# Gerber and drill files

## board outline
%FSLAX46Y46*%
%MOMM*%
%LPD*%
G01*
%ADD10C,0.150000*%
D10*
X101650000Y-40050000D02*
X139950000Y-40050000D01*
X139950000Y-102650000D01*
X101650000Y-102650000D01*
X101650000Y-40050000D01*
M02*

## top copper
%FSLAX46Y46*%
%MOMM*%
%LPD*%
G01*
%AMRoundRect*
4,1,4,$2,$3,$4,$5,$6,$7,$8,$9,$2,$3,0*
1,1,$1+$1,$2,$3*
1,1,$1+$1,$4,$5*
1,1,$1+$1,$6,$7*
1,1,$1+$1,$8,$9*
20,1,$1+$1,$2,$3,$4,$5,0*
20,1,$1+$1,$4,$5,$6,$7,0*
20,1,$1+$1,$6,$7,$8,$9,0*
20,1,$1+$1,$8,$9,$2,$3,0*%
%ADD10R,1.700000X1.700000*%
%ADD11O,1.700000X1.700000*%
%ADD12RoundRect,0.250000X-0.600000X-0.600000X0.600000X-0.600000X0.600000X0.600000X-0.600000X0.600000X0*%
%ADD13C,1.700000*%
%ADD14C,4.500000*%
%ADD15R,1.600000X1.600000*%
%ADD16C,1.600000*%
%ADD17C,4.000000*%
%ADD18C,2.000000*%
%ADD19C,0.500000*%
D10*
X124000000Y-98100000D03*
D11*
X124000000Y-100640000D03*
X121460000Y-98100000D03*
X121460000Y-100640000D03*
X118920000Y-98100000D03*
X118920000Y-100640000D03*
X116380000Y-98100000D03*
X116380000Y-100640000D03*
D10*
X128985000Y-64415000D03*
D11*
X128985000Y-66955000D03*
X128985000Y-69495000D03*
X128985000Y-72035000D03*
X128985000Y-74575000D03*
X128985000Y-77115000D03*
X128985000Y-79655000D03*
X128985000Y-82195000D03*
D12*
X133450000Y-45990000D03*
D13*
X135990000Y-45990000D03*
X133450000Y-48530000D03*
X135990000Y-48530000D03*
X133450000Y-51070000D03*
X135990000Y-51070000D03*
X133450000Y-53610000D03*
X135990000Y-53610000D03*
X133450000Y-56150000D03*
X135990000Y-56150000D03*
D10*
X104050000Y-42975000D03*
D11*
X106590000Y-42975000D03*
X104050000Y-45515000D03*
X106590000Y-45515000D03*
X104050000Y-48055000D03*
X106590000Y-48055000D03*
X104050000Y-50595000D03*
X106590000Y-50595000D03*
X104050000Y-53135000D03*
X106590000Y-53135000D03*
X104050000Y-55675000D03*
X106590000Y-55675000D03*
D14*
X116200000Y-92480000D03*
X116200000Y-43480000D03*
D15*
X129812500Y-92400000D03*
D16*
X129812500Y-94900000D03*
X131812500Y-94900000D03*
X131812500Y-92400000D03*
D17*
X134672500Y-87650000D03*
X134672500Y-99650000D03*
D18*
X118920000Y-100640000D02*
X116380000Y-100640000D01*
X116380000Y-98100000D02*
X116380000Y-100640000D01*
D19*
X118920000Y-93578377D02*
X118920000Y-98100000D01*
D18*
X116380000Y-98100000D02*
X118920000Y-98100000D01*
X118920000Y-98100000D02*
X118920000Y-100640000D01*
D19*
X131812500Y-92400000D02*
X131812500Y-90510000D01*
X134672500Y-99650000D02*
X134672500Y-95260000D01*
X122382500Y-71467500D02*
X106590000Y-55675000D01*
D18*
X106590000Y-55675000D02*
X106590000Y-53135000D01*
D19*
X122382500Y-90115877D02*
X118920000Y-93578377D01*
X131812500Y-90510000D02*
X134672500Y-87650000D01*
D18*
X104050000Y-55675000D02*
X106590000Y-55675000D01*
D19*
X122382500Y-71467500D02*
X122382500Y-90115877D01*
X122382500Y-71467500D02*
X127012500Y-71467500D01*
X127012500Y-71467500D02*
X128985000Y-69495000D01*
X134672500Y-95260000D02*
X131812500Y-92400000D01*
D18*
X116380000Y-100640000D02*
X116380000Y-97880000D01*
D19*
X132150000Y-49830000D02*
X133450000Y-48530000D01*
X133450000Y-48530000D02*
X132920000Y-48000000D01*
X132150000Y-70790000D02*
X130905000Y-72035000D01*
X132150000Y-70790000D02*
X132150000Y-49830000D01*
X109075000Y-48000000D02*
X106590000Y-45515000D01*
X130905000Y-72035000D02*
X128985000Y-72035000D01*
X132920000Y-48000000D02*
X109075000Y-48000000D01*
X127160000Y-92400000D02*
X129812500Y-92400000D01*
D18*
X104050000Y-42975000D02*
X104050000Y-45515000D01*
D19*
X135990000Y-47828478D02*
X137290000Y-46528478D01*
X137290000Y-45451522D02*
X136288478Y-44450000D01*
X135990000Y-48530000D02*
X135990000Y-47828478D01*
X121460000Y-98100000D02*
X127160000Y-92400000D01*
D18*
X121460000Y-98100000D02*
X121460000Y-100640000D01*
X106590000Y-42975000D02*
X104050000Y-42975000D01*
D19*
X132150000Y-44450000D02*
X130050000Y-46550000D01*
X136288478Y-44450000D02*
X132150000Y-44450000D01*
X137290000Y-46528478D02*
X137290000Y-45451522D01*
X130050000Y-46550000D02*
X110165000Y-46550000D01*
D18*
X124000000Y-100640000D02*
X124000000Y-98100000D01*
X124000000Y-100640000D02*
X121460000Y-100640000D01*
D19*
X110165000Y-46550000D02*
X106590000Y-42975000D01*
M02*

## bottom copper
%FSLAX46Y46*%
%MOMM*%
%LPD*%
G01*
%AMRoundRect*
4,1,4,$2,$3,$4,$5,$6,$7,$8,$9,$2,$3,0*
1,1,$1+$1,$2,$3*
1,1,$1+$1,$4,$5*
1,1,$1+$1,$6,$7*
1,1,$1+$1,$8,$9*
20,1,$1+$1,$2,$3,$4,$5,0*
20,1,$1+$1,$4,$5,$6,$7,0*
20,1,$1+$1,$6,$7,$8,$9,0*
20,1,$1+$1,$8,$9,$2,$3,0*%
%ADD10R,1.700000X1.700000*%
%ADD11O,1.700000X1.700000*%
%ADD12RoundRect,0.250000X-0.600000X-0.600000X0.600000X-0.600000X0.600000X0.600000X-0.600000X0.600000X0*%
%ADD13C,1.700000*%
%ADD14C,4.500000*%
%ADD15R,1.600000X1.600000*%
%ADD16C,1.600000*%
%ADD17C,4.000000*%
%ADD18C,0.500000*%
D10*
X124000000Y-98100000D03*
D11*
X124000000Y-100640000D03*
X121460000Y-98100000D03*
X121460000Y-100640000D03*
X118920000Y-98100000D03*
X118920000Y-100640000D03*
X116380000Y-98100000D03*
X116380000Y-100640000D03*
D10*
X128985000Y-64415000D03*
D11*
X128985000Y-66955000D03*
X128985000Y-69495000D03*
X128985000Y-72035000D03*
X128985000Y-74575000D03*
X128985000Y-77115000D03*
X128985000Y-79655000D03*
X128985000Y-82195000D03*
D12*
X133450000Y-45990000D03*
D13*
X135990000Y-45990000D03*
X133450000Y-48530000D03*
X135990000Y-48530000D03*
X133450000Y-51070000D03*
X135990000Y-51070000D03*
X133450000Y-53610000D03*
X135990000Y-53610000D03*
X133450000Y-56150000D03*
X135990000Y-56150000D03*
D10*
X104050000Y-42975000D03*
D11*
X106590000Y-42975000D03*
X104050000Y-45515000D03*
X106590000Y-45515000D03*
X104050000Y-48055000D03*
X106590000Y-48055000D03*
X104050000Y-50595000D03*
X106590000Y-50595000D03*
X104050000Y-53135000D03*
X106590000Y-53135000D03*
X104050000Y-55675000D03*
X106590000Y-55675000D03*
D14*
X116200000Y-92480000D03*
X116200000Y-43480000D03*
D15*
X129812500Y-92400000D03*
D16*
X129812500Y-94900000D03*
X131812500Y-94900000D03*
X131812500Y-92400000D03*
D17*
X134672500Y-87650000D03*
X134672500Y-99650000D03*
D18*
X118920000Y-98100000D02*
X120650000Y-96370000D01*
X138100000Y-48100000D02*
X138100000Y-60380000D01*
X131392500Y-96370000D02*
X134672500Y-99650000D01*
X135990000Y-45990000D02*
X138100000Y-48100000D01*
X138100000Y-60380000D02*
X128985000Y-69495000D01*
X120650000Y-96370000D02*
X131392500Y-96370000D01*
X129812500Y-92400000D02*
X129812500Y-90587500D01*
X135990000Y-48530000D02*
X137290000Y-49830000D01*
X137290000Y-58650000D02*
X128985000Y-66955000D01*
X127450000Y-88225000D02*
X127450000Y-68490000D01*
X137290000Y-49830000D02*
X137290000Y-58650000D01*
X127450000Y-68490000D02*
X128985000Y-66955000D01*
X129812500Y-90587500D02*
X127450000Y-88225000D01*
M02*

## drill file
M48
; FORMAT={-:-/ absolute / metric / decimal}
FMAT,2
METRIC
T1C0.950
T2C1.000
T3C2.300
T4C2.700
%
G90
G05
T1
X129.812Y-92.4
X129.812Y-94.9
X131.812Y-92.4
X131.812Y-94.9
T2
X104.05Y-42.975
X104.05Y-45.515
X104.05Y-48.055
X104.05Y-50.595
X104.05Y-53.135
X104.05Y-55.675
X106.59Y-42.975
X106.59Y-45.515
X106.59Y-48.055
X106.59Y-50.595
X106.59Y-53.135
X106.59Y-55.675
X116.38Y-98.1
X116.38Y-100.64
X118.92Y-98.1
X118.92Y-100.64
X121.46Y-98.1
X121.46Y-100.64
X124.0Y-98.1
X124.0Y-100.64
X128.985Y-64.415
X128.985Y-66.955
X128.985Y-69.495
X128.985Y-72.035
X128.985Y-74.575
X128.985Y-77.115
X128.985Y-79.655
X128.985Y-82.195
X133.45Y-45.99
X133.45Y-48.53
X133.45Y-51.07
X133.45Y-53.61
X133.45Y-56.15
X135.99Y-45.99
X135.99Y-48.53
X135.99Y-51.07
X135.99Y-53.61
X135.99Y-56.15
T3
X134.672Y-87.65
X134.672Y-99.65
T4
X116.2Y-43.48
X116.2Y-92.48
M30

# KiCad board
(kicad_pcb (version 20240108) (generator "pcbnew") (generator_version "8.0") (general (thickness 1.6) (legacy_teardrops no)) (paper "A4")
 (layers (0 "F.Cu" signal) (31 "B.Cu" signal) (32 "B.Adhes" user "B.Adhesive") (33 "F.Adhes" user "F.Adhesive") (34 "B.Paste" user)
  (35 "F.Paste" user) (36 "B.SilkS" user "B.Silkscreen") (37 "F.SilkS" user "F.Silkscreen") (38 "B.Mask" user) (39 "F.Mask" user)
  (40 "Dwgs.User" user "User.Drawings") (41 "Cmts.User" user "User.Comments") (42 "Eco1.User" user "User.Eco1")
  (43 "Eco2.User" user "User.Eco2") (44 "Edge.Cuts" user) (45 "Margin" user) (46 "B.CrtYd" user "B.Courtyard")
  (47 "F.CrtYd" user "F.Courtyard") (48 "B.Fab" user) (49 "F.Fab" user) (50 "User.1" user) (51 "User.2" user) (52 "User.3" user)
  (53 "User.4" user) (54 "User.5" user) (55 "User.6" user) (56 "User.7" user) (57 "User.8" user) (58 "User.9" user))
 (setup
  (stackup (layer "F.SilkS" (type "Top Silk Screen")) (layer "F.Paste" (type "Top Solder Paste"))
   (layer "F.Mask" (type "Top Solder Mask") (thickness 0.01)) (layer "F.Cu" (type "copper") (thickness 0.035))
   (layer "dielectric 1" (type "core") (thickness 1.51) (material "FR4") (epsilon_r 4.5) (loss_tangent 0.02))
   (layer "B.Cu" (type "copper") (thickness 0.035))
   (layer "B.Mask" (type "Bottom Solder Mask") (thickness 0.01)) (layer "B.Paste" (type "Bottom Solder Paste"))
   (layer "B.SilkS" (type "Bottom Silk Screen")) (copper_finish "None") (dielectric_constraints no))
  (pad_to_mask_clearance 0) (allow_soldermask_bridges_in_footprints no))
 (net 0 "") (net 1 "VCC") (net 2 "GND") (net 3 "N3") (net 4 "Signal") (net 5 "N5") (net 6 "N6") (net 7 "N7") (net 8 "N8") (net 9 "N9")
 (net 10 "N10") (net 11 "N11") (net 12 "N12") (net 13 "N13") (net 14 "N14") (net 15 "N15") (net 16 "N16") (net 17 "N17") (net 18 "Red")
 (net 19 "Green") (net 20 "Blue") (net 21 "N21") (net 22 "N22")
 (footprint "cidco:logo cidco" (layer "F.Cu") (at 113.75 73.78)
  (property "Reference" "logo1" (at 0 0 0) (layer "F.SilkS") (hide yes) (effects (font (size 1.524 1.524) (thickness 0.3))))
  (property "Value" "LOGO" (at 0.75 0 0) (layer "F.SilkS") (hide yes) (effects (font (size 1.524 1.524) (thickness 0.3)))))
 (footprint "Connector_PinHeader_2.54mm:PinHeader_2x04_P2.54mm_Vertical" (layer "F.Cu") (at 124 98.1 -90)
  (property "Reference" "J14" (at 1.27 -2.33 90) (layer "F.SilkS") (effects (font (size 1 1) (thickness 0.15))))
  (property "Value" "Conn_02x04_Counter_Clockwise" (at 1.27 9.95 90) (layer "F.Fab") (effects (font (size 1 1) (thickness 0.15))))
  (pad "1" thru_hole rect (at 0 0 270) (size 1.7 1.7) (drill 1) (layers "*.Cu" "*.Mask") (remove_unused_layers no) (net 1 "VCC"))
  (pad "2" thru_hole oval (at 2.54 0 270) (size 1.7 1.7) (drill 1) (layers "*.Cu" "*.Mask") (remove_unused_layers no) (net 1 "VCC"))
  (pad "3" thru_hole oval (at 0 2.54 270) (size 1.7 1.7) (drill 1) (layers "*.Cu" "*.Mask") (remove_unused_layers no) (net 1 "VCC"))
  (pad "4" thru_hole oval (at 2.54 2.54 270) (size 1.7 1.7) (drill 1) (layers "*.Cu" "*.Mask") (remove_unused_layers no) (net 1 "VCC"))
  (pad "5" thru_hole oval (at 0 5.08 270) (size 1.7 1.7) (drill 1) (layers "*.Cu" "*.Mask") (remove_unused_layers no) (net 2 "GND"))
  (pad "6" thru_hole oval (at 2.54 5.08 270) (size 1.7 1.7) (drill 1) (layers "*.Cu" "*.Mask") (remove_unused_layers no) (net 2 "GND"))
  (pad "7" thru_hole oval (at 0 7.62 270) (size 1.7 1.7) (drill 1) (layers "*.Cu" "*.Mask") (remove_unused_layers no) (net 2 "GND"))
  (pad "8" thru_hole oval (at 2.54 7.62 270) (size 1.7 1.7) (drill 1) (layers "*.Cu" "*.Mask") (remove_unused_layers no) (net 2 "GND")))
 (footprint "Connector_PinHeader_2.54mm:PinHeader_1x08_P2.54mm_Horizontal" (layer "F.Cu") (at 128.985 64.415)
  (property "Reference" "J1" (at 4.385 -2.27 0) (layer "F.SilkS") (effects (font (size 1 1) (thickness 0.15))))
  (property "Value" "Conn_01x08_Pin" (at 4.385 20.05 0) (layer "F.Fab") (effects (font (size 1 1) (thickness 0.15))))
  (pad "1" thru_hole rect (at 0 0) (size 1.7 1.7) (drill 1) (layers "*.Cu" "*.Mask") (remove_unused_layers no) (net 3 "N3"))
  (pad "2" thru_hole oval (at 0 2.54) (size 1.7 1.7) (drill 1) (layers "*.Cu" "*.Mask") (remove_unused_layers no) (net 1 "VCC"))
  (pad "3" thru_hole oval (at 0 5.08) (size 1.7 1.7) (drill 1) (layers "*.Cu" "*.Mask") (remove_unused_layers no) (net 2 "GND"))
  (pad "4" thru_hole oval (at 0 7.62) (size 1.7 1.7) (drill 1) (layers "*.Cu" "*.Mask") (remove_unused_layers no) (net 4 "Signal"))
  (pad "5" thru_hole oval (at 0 10.16) (size 1.7 1.7) (drill 1) (layers "*.Cu" "*.Mask") (remove_unused_layers no) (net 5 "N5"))
  (pad "6" thru_hole oval (at 0 12.7) (size 1.7 1.7) (drill 1) (layers "*.Cu" "*.Mask") (remove_unused_layers no) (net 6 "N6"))
  (pad "7" thru_hole oval (at 0 15.24) (size 1.7 1.7) (drill 1) (layers "*.Cu" "*.Mask") (remove_unused_layers no) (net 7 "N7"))
  (pad "8" thru_hole oval (at 0 17.78) (size 1.7 1.7) (drill 1) (layers "*.Cu" "*.Mask") (remove_unused_layers no) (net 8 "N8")))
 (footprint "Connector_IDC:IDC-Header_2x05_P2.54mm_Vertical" (layer "F.Cu") (at 133.45 45.99)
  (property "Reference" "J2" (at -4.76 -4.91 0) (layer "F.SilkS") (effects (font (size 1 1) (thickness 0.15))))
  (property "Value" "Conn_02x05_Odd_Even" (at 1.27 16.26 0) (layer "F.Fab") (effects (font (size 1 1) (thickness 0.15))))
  (pad "1" thru_hole roundrect (at 0 0) (size 1.7 1.7) (drill 1) (layers "*.Cu" "*.Mask") (remove_unused_layers no)
   (roundrect_rratio 0.147059) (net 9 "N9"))
  (pad "2" thru_hole circle (at 2.54 0) (size 1.7 1.7) (drill 1) (layers "*.Cu" "*.Mask") (remove_unused_layers no) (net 2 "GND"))
  (pad "3" thru_hole circle (at 0 2.54) (size 1.7 1.7) (drill 1) (layers "*.Cu" "*.Mask") (remove_unused_layers no) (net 4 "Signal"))
  (pad "4" thru_hole circle (at 2.54 2.54) (size 1.7 1.7) (drill 1) (layers "*.Cu" "*.Mask") (remove_unused_layers no) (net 1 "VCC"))
  (pad "5" thru_hole circle (at 0 5.08) (size 1.7 1.7) (drill 1) (layers "*.Cu" "*.Mask") (remove_unused_layers no) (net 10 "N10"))
  (pad "6" thru_hole circle (at 2.54 5.08) (size 1.7 1.7) (drill 1) (layers "*.Cu" "*.Mask") (remove_unused_layers no) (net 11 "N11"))
  (pad "7" thru_hole circle (at 0 7.62) (size 1.7 1.7) (drill 1) (layers "*.Cu" "*.Mask") (remove_unused_layers no) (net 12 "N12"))
  (pad "8" thru_hole circle (at 2.54 7.62) (size 1.7 1.7) (drill 1) (layers "*.Cu" "*.Mask") (remove_unused_layers no) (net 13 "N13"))
  (pad "9" thru_hole circle (at 0 10.16) (size 1.7 1.7) (drill 1) (layers "*.Cu" "*.Mask") (remove_unused_layers no) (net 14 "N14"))
  (pad "10" thru_hole circle (at 2.54 10.16) (size 1.7 1.7) (drill 1) (layers "*.Cu" "*.Mask") (remove_unused_layers no) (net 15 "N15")))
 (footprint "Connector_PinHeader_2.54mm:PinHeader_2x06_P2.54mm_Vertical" (layer "F.Cu") (at 104.05 42.975)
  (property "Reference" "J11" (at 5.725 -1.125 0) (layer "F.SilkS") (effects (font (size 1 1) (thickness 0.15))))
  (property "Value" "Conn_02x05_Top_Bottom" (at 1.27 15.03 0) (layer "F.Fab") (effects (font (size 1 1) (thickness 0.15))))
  (pad "1" thru_hole rect (at 0 0) (size 1.7 1.7) (drill 1) (layers "*.Cu" "*.Mask") (remove_unused_layers no) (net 1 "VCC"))
  (pad "2" thru_hole oval (at 2.54 0) (size 1.7 1.7) (drill 1) (layers "*.Cu" "*.Mask") (remove_unused_layers no) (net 1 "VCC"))
  (pad "3" thru_hole oval (at 0 2.54) (size 1.7 1.7) (drill 1) (layers "*.Cu" "*.Mask") (remove_unused_layers no) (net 1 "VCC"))
  (pad "4" thru_hole oval (at 2.54 2.54) (size 1.7 1.7) (drill 1) (layers "*.Cu" "*.Mask") (remove_unused_layers no) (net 4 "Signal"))
  (pad "5" thru_hole oval (at 0 5.08) (size 1.7 1.7) (drill 1) (layers "*.Cu" "*.Mask") (remove_unused_layers no) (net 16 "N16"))
  (pad "6" thru_hole oval (at 2.54 5.08) (size 1.7 1.7) (drill 1) (layers "*.Cu" "*.Mask") (remove_unused_layers no) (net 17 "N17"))
  (pad "7" thru_hole oval (at 0 7.62) (size 1.7 1.7) (drill 1) (layers "*.Cu" "*.Mask") (remove_unused_layers no) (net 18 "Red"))
  (pad "8" thru_hole oval (at 2.54 7.62) (size 1.7 1.7) (drill 1) (layers "*.Cu" "*.Mask") (remove_unused_layers no) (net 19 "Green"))
  (pad "9" thru_hole oval (at 0 10.16) (size 1.7 1.7) (drill 1) (layers "*.Cu" "*.Mask") (remove_unused_layers no) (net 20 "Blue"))
  (pad "10" thru_hole oval (at 2.54 10.16) (size 1.7 1.7) (drill 1) (layers "*.Cu" "*.Mask") (remove_unused_layers no) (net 2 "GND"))
  (pad "11" thru_hole oval (at 0 12.7) (size 1.7 1.7) (drill 1) (layers "*.Cu" "*.Mask") (remove_unused_layers no) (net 2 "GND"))
  (pad "12" thru_hole oval (at 2.54 12.7) (size 1.7 1.7) (drill 1) (layers "*.Cu" "*.Mask") (remove_unused_layers no) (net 2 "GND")))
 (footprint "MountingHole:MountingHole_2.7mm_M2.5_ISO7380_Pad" (layer "F.Cu") (at 116.2 92.48)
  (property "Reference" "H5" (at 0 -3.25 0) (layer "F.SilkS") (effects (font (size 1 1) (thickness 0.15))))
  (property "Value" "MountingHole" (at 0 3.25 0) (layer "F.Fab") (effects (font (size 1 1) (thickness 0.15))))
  (pad "1" thru_hole circle (at 0 0) (size 4.5 4.5) (drill 2.7) (layers "*.Cu" "*.Mask") (remove_unused_layers no)))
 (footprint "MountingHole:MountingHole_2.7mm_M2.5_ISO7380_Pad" (layer "F.Cu") (at 116.2 43.48)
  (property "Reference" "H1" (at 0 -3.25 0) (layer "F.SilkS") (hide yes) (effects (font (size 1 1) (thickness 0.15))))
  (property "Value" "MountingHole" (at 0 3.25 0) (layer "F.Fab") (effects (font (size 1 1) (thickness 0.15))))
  (pad "1" thru_hole circle (at 0 0) (size 4.5 4.5) (drill 2.7) (layers "*.Cu" "*.Mask") (remove_unused_layers no)))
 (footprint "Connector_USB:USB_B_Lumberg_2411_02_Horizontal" (layer "F.Cu") (at 129.8125 92.4)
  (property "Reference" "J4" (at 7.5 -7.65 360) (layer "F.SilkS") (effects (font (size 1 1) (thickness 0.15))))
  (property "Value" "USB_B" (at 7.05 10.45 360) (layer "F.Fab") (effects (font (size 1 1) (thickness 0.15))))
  (pad "1" thru_hole rect (at 0 0 90) (size 1.6 1.6) (drill 0.95) (layers "*.Cu" "*.Mask") (remove_unused_layers no) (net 1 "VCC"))
  (pad "2" thru_hole circle (at 0 2.5 90) (size 1.6 1.6) (drill 0.95) (layers "*.Cu" "*.Mask") (remove_unused_layers no) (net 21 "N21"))
  (pad "3" thru_hole circle (at 2 2.5 90) (size 1.6 1.6) (drill 0.95) (layers "*.Cu" "*.Mask") (remove_unused_layers no) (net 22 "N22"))
  (pad "4" thru_hole circle (at 2 0 90) (size 1.6 1.6) (drill 0.95) (layers "*.Cu" "*.Mask") (remove_unused_layers no) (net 2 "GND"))
  (pad "5" thru_hole circle (at 4.86 -4.75 90) (size 4 4) (drill 2.3) (layers "*.Cu" "*.Mask") (remove_unused_layers no) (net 2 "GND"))
  (pad "5" thru_hole circle (at 4.86 7.25 90) (size 4 4) (drill 2.3) (layers "*.Cu" "*.Mask") (remove_unused_layers no) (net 2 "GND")))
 (gr_rect (start 101.65 40.05) (end 139.95 102.65) (stroke (width 0.15) (type default)) (fill none) (layer "Edge.Cuts"))
 (segment (start 118.92 100.64) (end 116.38 100.64) (width 2) (layer "F.Cu") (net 2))
 (segment (start 116.38 98.1) (end 116.38 100.64) (width 2) (layer "F.Cu") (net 2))
 (segment (start 118.92 93.578377) (end 118.92 98.1) (width 0.5) (layer "F.Cu") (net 2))
 (segment (start 116.38 98.1) (end 118.92 98.1) (width 2) (layer "F.Cu") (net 2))
 (segment (start 118.92 98.1) (end 118.92 100.64) (width 2) (layer "F.Cu") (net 2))
 (segment (start 131.8125 92.4) (end 131.8125 90.51) (width 0.5) (layer "F.Cu") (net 2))
 (segment (start 134.6725 99.65) (end 134.6725 95.26) (width 0.5) (layer "F.Cu") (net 2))
 (segment (start 122.3825 71.4675) (end 106.59 55.675) (width 0.5) (layer "F.Cu") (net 2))
 (segment (start 106.59 55.675) (end 106.59 53.135) (width 2) (layer "F.Cu") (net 2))
 (segment (start 122.3825 90.115877) (end 118.92 93.578377) (width 0.5) (layer "F.Cu") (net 2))
 (segment (start 131.8125 90.51) (end 134.6725 87.65) (width 0.5) (layer "F.Cu") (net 2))
 (segment (start 104.05 55.675) (end 106.59 55.675) (width 2) (layer "F.Cu") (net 2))
 (segment (start 122.3825 71.4675) (end 122.3825 90.115877) (width 0.5) (layer "F.Cu") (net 2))
 (segment (start 122.3825 71.4675) (end 127.0125 71.4675) (width 0.5) (layer "F.Cu") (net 2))
 (segment (start 127.0125 71.4675) (end 128.985 69.495) (width 0.5) (layer "F.Cu") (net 2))
 (segment (start 134.6725 95.26) (end 131.8125 92.4) (width 0.5) (layer "F.Cu") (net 2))
 (segment (start 116.38 100.64) (end 116.38 97.88) (width 2) (layer "F.Cu") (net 2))
 (segment (start 118.92 98.1) (end 120.65 96.37) (width 0.5) (layer "B.Cu") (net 2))
 (segment (start 138.1 48.1) (end 138.1 60.38) (width 0.5) (layer "B.Cu") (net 2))
 (segment (start 131.3925 96.37) (end 134.6725 99.65) (width 0.5) (layer "B.Cu") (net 2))
 (segment (start 135.99 45.99) (end 138.1 48.1) (width 0.5) (layer "B.Cu") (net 2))
 (segment (start 138.1 60.38) (end 128.985 69.495) (width 0.5) (layer "B.Cu") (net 2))
 (segment (start 120.65 96.37) (end 131.3925 96.37) (width 0.5) (layer "B.Cu") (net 2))
 (segment (start 132.15 49.83) (end 133.45 48.53) (width 0.5) (layer "F.Cu") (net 4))
 (segment (start 133.45 48.53) (end 132.92 48) (width 0.5) (layer "F.Cu") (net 4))
 (segment (start 132.15 70.79) (end 130.905 72.035) (width 0.5) (layer "F.Cu") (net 4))
 (segment (start 132.15 70.79) (end 132.15 49.83) (width 0.5) (layer "F.Cu") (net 4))
 (segment (start 109.075 48) (end 106.59 45.515) (width 0.5) (layer "F.Cu") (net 4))
 (segment (start 130.905 72.035) (end 128.985 72.035) (width 0.5) (layer "F.Cu") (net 4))
 (segment (start 132.92 48) (end 109.075 48) (width 0.5) (layer "F.Cu") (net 4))
 (segment (start 127.16 92.4) (end 129.8125 92.4) (width 0.5) (layer "F.Cu") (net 1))
 (segment (start 104.05 42.975) (end 104.05 45.515) (width 2) (layer "F.Cu") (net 1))
 (segment (start 135.99 47.828478) (end 137.29 46.528478) (width 0.5) (layer "F.Cu") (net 1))
 (segment (start 137.29 45.451522) (end 136.288478 44.45) (width 0.5) (layer "F.Cu") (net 1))
 (segment (start 135.99 48.53) (end 135.99 47.828478) (width 0.5) (layer "F.Cu") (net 1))
 (segment (start 121.46 98.1) (end 127.16 92.4) (width 0.5) (layer "F.Cu") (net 1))
 (segment (start 121.46 98.1) (end 121.46 100.64) (width 2) (layer "F.Cu") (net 1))
 (segment (start 106.59 42.975) (end 104.05 42.975) (width 2) (layer "F.Cu") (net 1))
 (segment (start 132.15 44.45) (end 130.05 46.55) (width 0.5) (layer "F.Cu") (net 1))
 (segment (start 136.288478 44.45) (end 132.15 44.45) (width 0.5) (layer "F.Cu") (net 1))
 (segment (start 137.29 46.528478) (end 137.29 45.451522) (width 0.5) (layer "F.Cu") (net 1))
 (segment (start 130.05 46.55) (end 110.165 46.55) (width 0.5) (layer "F.Cu") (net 1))
 (segment (start 124 100.64) (end 124 98.1) (width 2) (layer "F.Cu") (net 1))
 (segment (start 124 100.64) (end 121.46 100.64) (width 2) (layer "F.Cu") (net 1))
 (segment (start 110.165 46.55) (end 106.59 42.975) (width 0.5) (layer "F.Cu") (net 1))
 (segment (start 129.8125 92.4) (end 129.8125 90.5875) (width 0.5) (layer "B.Cu") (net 1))
 (segment (start 135.99 48.53) (end 137.29 49.83) (width 0.5) (layer "B.Cu") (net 1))
 (segment (start 137.29 58.65) (end 128.985 66.955) (width 0.5) (layer "B.Cu") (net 1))
 (segment (start 127.45 88.225) (end 127.45 68.49) (width 0.5) (layer "B.Cu") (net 1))
 (segment (start 137.29 49.83) (end 137.29 58.65) (width 0.5) (layer "B.Cu") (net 1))
 (segment (start 127.45 68.49) (end 128.985 66.955) (width 0.5) (layer "B.Cu") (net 1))
 (segment (start 129.8125 90.5875) (end 127.45 88.225) (width 0.5) (layer "B.Cu") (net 1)))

